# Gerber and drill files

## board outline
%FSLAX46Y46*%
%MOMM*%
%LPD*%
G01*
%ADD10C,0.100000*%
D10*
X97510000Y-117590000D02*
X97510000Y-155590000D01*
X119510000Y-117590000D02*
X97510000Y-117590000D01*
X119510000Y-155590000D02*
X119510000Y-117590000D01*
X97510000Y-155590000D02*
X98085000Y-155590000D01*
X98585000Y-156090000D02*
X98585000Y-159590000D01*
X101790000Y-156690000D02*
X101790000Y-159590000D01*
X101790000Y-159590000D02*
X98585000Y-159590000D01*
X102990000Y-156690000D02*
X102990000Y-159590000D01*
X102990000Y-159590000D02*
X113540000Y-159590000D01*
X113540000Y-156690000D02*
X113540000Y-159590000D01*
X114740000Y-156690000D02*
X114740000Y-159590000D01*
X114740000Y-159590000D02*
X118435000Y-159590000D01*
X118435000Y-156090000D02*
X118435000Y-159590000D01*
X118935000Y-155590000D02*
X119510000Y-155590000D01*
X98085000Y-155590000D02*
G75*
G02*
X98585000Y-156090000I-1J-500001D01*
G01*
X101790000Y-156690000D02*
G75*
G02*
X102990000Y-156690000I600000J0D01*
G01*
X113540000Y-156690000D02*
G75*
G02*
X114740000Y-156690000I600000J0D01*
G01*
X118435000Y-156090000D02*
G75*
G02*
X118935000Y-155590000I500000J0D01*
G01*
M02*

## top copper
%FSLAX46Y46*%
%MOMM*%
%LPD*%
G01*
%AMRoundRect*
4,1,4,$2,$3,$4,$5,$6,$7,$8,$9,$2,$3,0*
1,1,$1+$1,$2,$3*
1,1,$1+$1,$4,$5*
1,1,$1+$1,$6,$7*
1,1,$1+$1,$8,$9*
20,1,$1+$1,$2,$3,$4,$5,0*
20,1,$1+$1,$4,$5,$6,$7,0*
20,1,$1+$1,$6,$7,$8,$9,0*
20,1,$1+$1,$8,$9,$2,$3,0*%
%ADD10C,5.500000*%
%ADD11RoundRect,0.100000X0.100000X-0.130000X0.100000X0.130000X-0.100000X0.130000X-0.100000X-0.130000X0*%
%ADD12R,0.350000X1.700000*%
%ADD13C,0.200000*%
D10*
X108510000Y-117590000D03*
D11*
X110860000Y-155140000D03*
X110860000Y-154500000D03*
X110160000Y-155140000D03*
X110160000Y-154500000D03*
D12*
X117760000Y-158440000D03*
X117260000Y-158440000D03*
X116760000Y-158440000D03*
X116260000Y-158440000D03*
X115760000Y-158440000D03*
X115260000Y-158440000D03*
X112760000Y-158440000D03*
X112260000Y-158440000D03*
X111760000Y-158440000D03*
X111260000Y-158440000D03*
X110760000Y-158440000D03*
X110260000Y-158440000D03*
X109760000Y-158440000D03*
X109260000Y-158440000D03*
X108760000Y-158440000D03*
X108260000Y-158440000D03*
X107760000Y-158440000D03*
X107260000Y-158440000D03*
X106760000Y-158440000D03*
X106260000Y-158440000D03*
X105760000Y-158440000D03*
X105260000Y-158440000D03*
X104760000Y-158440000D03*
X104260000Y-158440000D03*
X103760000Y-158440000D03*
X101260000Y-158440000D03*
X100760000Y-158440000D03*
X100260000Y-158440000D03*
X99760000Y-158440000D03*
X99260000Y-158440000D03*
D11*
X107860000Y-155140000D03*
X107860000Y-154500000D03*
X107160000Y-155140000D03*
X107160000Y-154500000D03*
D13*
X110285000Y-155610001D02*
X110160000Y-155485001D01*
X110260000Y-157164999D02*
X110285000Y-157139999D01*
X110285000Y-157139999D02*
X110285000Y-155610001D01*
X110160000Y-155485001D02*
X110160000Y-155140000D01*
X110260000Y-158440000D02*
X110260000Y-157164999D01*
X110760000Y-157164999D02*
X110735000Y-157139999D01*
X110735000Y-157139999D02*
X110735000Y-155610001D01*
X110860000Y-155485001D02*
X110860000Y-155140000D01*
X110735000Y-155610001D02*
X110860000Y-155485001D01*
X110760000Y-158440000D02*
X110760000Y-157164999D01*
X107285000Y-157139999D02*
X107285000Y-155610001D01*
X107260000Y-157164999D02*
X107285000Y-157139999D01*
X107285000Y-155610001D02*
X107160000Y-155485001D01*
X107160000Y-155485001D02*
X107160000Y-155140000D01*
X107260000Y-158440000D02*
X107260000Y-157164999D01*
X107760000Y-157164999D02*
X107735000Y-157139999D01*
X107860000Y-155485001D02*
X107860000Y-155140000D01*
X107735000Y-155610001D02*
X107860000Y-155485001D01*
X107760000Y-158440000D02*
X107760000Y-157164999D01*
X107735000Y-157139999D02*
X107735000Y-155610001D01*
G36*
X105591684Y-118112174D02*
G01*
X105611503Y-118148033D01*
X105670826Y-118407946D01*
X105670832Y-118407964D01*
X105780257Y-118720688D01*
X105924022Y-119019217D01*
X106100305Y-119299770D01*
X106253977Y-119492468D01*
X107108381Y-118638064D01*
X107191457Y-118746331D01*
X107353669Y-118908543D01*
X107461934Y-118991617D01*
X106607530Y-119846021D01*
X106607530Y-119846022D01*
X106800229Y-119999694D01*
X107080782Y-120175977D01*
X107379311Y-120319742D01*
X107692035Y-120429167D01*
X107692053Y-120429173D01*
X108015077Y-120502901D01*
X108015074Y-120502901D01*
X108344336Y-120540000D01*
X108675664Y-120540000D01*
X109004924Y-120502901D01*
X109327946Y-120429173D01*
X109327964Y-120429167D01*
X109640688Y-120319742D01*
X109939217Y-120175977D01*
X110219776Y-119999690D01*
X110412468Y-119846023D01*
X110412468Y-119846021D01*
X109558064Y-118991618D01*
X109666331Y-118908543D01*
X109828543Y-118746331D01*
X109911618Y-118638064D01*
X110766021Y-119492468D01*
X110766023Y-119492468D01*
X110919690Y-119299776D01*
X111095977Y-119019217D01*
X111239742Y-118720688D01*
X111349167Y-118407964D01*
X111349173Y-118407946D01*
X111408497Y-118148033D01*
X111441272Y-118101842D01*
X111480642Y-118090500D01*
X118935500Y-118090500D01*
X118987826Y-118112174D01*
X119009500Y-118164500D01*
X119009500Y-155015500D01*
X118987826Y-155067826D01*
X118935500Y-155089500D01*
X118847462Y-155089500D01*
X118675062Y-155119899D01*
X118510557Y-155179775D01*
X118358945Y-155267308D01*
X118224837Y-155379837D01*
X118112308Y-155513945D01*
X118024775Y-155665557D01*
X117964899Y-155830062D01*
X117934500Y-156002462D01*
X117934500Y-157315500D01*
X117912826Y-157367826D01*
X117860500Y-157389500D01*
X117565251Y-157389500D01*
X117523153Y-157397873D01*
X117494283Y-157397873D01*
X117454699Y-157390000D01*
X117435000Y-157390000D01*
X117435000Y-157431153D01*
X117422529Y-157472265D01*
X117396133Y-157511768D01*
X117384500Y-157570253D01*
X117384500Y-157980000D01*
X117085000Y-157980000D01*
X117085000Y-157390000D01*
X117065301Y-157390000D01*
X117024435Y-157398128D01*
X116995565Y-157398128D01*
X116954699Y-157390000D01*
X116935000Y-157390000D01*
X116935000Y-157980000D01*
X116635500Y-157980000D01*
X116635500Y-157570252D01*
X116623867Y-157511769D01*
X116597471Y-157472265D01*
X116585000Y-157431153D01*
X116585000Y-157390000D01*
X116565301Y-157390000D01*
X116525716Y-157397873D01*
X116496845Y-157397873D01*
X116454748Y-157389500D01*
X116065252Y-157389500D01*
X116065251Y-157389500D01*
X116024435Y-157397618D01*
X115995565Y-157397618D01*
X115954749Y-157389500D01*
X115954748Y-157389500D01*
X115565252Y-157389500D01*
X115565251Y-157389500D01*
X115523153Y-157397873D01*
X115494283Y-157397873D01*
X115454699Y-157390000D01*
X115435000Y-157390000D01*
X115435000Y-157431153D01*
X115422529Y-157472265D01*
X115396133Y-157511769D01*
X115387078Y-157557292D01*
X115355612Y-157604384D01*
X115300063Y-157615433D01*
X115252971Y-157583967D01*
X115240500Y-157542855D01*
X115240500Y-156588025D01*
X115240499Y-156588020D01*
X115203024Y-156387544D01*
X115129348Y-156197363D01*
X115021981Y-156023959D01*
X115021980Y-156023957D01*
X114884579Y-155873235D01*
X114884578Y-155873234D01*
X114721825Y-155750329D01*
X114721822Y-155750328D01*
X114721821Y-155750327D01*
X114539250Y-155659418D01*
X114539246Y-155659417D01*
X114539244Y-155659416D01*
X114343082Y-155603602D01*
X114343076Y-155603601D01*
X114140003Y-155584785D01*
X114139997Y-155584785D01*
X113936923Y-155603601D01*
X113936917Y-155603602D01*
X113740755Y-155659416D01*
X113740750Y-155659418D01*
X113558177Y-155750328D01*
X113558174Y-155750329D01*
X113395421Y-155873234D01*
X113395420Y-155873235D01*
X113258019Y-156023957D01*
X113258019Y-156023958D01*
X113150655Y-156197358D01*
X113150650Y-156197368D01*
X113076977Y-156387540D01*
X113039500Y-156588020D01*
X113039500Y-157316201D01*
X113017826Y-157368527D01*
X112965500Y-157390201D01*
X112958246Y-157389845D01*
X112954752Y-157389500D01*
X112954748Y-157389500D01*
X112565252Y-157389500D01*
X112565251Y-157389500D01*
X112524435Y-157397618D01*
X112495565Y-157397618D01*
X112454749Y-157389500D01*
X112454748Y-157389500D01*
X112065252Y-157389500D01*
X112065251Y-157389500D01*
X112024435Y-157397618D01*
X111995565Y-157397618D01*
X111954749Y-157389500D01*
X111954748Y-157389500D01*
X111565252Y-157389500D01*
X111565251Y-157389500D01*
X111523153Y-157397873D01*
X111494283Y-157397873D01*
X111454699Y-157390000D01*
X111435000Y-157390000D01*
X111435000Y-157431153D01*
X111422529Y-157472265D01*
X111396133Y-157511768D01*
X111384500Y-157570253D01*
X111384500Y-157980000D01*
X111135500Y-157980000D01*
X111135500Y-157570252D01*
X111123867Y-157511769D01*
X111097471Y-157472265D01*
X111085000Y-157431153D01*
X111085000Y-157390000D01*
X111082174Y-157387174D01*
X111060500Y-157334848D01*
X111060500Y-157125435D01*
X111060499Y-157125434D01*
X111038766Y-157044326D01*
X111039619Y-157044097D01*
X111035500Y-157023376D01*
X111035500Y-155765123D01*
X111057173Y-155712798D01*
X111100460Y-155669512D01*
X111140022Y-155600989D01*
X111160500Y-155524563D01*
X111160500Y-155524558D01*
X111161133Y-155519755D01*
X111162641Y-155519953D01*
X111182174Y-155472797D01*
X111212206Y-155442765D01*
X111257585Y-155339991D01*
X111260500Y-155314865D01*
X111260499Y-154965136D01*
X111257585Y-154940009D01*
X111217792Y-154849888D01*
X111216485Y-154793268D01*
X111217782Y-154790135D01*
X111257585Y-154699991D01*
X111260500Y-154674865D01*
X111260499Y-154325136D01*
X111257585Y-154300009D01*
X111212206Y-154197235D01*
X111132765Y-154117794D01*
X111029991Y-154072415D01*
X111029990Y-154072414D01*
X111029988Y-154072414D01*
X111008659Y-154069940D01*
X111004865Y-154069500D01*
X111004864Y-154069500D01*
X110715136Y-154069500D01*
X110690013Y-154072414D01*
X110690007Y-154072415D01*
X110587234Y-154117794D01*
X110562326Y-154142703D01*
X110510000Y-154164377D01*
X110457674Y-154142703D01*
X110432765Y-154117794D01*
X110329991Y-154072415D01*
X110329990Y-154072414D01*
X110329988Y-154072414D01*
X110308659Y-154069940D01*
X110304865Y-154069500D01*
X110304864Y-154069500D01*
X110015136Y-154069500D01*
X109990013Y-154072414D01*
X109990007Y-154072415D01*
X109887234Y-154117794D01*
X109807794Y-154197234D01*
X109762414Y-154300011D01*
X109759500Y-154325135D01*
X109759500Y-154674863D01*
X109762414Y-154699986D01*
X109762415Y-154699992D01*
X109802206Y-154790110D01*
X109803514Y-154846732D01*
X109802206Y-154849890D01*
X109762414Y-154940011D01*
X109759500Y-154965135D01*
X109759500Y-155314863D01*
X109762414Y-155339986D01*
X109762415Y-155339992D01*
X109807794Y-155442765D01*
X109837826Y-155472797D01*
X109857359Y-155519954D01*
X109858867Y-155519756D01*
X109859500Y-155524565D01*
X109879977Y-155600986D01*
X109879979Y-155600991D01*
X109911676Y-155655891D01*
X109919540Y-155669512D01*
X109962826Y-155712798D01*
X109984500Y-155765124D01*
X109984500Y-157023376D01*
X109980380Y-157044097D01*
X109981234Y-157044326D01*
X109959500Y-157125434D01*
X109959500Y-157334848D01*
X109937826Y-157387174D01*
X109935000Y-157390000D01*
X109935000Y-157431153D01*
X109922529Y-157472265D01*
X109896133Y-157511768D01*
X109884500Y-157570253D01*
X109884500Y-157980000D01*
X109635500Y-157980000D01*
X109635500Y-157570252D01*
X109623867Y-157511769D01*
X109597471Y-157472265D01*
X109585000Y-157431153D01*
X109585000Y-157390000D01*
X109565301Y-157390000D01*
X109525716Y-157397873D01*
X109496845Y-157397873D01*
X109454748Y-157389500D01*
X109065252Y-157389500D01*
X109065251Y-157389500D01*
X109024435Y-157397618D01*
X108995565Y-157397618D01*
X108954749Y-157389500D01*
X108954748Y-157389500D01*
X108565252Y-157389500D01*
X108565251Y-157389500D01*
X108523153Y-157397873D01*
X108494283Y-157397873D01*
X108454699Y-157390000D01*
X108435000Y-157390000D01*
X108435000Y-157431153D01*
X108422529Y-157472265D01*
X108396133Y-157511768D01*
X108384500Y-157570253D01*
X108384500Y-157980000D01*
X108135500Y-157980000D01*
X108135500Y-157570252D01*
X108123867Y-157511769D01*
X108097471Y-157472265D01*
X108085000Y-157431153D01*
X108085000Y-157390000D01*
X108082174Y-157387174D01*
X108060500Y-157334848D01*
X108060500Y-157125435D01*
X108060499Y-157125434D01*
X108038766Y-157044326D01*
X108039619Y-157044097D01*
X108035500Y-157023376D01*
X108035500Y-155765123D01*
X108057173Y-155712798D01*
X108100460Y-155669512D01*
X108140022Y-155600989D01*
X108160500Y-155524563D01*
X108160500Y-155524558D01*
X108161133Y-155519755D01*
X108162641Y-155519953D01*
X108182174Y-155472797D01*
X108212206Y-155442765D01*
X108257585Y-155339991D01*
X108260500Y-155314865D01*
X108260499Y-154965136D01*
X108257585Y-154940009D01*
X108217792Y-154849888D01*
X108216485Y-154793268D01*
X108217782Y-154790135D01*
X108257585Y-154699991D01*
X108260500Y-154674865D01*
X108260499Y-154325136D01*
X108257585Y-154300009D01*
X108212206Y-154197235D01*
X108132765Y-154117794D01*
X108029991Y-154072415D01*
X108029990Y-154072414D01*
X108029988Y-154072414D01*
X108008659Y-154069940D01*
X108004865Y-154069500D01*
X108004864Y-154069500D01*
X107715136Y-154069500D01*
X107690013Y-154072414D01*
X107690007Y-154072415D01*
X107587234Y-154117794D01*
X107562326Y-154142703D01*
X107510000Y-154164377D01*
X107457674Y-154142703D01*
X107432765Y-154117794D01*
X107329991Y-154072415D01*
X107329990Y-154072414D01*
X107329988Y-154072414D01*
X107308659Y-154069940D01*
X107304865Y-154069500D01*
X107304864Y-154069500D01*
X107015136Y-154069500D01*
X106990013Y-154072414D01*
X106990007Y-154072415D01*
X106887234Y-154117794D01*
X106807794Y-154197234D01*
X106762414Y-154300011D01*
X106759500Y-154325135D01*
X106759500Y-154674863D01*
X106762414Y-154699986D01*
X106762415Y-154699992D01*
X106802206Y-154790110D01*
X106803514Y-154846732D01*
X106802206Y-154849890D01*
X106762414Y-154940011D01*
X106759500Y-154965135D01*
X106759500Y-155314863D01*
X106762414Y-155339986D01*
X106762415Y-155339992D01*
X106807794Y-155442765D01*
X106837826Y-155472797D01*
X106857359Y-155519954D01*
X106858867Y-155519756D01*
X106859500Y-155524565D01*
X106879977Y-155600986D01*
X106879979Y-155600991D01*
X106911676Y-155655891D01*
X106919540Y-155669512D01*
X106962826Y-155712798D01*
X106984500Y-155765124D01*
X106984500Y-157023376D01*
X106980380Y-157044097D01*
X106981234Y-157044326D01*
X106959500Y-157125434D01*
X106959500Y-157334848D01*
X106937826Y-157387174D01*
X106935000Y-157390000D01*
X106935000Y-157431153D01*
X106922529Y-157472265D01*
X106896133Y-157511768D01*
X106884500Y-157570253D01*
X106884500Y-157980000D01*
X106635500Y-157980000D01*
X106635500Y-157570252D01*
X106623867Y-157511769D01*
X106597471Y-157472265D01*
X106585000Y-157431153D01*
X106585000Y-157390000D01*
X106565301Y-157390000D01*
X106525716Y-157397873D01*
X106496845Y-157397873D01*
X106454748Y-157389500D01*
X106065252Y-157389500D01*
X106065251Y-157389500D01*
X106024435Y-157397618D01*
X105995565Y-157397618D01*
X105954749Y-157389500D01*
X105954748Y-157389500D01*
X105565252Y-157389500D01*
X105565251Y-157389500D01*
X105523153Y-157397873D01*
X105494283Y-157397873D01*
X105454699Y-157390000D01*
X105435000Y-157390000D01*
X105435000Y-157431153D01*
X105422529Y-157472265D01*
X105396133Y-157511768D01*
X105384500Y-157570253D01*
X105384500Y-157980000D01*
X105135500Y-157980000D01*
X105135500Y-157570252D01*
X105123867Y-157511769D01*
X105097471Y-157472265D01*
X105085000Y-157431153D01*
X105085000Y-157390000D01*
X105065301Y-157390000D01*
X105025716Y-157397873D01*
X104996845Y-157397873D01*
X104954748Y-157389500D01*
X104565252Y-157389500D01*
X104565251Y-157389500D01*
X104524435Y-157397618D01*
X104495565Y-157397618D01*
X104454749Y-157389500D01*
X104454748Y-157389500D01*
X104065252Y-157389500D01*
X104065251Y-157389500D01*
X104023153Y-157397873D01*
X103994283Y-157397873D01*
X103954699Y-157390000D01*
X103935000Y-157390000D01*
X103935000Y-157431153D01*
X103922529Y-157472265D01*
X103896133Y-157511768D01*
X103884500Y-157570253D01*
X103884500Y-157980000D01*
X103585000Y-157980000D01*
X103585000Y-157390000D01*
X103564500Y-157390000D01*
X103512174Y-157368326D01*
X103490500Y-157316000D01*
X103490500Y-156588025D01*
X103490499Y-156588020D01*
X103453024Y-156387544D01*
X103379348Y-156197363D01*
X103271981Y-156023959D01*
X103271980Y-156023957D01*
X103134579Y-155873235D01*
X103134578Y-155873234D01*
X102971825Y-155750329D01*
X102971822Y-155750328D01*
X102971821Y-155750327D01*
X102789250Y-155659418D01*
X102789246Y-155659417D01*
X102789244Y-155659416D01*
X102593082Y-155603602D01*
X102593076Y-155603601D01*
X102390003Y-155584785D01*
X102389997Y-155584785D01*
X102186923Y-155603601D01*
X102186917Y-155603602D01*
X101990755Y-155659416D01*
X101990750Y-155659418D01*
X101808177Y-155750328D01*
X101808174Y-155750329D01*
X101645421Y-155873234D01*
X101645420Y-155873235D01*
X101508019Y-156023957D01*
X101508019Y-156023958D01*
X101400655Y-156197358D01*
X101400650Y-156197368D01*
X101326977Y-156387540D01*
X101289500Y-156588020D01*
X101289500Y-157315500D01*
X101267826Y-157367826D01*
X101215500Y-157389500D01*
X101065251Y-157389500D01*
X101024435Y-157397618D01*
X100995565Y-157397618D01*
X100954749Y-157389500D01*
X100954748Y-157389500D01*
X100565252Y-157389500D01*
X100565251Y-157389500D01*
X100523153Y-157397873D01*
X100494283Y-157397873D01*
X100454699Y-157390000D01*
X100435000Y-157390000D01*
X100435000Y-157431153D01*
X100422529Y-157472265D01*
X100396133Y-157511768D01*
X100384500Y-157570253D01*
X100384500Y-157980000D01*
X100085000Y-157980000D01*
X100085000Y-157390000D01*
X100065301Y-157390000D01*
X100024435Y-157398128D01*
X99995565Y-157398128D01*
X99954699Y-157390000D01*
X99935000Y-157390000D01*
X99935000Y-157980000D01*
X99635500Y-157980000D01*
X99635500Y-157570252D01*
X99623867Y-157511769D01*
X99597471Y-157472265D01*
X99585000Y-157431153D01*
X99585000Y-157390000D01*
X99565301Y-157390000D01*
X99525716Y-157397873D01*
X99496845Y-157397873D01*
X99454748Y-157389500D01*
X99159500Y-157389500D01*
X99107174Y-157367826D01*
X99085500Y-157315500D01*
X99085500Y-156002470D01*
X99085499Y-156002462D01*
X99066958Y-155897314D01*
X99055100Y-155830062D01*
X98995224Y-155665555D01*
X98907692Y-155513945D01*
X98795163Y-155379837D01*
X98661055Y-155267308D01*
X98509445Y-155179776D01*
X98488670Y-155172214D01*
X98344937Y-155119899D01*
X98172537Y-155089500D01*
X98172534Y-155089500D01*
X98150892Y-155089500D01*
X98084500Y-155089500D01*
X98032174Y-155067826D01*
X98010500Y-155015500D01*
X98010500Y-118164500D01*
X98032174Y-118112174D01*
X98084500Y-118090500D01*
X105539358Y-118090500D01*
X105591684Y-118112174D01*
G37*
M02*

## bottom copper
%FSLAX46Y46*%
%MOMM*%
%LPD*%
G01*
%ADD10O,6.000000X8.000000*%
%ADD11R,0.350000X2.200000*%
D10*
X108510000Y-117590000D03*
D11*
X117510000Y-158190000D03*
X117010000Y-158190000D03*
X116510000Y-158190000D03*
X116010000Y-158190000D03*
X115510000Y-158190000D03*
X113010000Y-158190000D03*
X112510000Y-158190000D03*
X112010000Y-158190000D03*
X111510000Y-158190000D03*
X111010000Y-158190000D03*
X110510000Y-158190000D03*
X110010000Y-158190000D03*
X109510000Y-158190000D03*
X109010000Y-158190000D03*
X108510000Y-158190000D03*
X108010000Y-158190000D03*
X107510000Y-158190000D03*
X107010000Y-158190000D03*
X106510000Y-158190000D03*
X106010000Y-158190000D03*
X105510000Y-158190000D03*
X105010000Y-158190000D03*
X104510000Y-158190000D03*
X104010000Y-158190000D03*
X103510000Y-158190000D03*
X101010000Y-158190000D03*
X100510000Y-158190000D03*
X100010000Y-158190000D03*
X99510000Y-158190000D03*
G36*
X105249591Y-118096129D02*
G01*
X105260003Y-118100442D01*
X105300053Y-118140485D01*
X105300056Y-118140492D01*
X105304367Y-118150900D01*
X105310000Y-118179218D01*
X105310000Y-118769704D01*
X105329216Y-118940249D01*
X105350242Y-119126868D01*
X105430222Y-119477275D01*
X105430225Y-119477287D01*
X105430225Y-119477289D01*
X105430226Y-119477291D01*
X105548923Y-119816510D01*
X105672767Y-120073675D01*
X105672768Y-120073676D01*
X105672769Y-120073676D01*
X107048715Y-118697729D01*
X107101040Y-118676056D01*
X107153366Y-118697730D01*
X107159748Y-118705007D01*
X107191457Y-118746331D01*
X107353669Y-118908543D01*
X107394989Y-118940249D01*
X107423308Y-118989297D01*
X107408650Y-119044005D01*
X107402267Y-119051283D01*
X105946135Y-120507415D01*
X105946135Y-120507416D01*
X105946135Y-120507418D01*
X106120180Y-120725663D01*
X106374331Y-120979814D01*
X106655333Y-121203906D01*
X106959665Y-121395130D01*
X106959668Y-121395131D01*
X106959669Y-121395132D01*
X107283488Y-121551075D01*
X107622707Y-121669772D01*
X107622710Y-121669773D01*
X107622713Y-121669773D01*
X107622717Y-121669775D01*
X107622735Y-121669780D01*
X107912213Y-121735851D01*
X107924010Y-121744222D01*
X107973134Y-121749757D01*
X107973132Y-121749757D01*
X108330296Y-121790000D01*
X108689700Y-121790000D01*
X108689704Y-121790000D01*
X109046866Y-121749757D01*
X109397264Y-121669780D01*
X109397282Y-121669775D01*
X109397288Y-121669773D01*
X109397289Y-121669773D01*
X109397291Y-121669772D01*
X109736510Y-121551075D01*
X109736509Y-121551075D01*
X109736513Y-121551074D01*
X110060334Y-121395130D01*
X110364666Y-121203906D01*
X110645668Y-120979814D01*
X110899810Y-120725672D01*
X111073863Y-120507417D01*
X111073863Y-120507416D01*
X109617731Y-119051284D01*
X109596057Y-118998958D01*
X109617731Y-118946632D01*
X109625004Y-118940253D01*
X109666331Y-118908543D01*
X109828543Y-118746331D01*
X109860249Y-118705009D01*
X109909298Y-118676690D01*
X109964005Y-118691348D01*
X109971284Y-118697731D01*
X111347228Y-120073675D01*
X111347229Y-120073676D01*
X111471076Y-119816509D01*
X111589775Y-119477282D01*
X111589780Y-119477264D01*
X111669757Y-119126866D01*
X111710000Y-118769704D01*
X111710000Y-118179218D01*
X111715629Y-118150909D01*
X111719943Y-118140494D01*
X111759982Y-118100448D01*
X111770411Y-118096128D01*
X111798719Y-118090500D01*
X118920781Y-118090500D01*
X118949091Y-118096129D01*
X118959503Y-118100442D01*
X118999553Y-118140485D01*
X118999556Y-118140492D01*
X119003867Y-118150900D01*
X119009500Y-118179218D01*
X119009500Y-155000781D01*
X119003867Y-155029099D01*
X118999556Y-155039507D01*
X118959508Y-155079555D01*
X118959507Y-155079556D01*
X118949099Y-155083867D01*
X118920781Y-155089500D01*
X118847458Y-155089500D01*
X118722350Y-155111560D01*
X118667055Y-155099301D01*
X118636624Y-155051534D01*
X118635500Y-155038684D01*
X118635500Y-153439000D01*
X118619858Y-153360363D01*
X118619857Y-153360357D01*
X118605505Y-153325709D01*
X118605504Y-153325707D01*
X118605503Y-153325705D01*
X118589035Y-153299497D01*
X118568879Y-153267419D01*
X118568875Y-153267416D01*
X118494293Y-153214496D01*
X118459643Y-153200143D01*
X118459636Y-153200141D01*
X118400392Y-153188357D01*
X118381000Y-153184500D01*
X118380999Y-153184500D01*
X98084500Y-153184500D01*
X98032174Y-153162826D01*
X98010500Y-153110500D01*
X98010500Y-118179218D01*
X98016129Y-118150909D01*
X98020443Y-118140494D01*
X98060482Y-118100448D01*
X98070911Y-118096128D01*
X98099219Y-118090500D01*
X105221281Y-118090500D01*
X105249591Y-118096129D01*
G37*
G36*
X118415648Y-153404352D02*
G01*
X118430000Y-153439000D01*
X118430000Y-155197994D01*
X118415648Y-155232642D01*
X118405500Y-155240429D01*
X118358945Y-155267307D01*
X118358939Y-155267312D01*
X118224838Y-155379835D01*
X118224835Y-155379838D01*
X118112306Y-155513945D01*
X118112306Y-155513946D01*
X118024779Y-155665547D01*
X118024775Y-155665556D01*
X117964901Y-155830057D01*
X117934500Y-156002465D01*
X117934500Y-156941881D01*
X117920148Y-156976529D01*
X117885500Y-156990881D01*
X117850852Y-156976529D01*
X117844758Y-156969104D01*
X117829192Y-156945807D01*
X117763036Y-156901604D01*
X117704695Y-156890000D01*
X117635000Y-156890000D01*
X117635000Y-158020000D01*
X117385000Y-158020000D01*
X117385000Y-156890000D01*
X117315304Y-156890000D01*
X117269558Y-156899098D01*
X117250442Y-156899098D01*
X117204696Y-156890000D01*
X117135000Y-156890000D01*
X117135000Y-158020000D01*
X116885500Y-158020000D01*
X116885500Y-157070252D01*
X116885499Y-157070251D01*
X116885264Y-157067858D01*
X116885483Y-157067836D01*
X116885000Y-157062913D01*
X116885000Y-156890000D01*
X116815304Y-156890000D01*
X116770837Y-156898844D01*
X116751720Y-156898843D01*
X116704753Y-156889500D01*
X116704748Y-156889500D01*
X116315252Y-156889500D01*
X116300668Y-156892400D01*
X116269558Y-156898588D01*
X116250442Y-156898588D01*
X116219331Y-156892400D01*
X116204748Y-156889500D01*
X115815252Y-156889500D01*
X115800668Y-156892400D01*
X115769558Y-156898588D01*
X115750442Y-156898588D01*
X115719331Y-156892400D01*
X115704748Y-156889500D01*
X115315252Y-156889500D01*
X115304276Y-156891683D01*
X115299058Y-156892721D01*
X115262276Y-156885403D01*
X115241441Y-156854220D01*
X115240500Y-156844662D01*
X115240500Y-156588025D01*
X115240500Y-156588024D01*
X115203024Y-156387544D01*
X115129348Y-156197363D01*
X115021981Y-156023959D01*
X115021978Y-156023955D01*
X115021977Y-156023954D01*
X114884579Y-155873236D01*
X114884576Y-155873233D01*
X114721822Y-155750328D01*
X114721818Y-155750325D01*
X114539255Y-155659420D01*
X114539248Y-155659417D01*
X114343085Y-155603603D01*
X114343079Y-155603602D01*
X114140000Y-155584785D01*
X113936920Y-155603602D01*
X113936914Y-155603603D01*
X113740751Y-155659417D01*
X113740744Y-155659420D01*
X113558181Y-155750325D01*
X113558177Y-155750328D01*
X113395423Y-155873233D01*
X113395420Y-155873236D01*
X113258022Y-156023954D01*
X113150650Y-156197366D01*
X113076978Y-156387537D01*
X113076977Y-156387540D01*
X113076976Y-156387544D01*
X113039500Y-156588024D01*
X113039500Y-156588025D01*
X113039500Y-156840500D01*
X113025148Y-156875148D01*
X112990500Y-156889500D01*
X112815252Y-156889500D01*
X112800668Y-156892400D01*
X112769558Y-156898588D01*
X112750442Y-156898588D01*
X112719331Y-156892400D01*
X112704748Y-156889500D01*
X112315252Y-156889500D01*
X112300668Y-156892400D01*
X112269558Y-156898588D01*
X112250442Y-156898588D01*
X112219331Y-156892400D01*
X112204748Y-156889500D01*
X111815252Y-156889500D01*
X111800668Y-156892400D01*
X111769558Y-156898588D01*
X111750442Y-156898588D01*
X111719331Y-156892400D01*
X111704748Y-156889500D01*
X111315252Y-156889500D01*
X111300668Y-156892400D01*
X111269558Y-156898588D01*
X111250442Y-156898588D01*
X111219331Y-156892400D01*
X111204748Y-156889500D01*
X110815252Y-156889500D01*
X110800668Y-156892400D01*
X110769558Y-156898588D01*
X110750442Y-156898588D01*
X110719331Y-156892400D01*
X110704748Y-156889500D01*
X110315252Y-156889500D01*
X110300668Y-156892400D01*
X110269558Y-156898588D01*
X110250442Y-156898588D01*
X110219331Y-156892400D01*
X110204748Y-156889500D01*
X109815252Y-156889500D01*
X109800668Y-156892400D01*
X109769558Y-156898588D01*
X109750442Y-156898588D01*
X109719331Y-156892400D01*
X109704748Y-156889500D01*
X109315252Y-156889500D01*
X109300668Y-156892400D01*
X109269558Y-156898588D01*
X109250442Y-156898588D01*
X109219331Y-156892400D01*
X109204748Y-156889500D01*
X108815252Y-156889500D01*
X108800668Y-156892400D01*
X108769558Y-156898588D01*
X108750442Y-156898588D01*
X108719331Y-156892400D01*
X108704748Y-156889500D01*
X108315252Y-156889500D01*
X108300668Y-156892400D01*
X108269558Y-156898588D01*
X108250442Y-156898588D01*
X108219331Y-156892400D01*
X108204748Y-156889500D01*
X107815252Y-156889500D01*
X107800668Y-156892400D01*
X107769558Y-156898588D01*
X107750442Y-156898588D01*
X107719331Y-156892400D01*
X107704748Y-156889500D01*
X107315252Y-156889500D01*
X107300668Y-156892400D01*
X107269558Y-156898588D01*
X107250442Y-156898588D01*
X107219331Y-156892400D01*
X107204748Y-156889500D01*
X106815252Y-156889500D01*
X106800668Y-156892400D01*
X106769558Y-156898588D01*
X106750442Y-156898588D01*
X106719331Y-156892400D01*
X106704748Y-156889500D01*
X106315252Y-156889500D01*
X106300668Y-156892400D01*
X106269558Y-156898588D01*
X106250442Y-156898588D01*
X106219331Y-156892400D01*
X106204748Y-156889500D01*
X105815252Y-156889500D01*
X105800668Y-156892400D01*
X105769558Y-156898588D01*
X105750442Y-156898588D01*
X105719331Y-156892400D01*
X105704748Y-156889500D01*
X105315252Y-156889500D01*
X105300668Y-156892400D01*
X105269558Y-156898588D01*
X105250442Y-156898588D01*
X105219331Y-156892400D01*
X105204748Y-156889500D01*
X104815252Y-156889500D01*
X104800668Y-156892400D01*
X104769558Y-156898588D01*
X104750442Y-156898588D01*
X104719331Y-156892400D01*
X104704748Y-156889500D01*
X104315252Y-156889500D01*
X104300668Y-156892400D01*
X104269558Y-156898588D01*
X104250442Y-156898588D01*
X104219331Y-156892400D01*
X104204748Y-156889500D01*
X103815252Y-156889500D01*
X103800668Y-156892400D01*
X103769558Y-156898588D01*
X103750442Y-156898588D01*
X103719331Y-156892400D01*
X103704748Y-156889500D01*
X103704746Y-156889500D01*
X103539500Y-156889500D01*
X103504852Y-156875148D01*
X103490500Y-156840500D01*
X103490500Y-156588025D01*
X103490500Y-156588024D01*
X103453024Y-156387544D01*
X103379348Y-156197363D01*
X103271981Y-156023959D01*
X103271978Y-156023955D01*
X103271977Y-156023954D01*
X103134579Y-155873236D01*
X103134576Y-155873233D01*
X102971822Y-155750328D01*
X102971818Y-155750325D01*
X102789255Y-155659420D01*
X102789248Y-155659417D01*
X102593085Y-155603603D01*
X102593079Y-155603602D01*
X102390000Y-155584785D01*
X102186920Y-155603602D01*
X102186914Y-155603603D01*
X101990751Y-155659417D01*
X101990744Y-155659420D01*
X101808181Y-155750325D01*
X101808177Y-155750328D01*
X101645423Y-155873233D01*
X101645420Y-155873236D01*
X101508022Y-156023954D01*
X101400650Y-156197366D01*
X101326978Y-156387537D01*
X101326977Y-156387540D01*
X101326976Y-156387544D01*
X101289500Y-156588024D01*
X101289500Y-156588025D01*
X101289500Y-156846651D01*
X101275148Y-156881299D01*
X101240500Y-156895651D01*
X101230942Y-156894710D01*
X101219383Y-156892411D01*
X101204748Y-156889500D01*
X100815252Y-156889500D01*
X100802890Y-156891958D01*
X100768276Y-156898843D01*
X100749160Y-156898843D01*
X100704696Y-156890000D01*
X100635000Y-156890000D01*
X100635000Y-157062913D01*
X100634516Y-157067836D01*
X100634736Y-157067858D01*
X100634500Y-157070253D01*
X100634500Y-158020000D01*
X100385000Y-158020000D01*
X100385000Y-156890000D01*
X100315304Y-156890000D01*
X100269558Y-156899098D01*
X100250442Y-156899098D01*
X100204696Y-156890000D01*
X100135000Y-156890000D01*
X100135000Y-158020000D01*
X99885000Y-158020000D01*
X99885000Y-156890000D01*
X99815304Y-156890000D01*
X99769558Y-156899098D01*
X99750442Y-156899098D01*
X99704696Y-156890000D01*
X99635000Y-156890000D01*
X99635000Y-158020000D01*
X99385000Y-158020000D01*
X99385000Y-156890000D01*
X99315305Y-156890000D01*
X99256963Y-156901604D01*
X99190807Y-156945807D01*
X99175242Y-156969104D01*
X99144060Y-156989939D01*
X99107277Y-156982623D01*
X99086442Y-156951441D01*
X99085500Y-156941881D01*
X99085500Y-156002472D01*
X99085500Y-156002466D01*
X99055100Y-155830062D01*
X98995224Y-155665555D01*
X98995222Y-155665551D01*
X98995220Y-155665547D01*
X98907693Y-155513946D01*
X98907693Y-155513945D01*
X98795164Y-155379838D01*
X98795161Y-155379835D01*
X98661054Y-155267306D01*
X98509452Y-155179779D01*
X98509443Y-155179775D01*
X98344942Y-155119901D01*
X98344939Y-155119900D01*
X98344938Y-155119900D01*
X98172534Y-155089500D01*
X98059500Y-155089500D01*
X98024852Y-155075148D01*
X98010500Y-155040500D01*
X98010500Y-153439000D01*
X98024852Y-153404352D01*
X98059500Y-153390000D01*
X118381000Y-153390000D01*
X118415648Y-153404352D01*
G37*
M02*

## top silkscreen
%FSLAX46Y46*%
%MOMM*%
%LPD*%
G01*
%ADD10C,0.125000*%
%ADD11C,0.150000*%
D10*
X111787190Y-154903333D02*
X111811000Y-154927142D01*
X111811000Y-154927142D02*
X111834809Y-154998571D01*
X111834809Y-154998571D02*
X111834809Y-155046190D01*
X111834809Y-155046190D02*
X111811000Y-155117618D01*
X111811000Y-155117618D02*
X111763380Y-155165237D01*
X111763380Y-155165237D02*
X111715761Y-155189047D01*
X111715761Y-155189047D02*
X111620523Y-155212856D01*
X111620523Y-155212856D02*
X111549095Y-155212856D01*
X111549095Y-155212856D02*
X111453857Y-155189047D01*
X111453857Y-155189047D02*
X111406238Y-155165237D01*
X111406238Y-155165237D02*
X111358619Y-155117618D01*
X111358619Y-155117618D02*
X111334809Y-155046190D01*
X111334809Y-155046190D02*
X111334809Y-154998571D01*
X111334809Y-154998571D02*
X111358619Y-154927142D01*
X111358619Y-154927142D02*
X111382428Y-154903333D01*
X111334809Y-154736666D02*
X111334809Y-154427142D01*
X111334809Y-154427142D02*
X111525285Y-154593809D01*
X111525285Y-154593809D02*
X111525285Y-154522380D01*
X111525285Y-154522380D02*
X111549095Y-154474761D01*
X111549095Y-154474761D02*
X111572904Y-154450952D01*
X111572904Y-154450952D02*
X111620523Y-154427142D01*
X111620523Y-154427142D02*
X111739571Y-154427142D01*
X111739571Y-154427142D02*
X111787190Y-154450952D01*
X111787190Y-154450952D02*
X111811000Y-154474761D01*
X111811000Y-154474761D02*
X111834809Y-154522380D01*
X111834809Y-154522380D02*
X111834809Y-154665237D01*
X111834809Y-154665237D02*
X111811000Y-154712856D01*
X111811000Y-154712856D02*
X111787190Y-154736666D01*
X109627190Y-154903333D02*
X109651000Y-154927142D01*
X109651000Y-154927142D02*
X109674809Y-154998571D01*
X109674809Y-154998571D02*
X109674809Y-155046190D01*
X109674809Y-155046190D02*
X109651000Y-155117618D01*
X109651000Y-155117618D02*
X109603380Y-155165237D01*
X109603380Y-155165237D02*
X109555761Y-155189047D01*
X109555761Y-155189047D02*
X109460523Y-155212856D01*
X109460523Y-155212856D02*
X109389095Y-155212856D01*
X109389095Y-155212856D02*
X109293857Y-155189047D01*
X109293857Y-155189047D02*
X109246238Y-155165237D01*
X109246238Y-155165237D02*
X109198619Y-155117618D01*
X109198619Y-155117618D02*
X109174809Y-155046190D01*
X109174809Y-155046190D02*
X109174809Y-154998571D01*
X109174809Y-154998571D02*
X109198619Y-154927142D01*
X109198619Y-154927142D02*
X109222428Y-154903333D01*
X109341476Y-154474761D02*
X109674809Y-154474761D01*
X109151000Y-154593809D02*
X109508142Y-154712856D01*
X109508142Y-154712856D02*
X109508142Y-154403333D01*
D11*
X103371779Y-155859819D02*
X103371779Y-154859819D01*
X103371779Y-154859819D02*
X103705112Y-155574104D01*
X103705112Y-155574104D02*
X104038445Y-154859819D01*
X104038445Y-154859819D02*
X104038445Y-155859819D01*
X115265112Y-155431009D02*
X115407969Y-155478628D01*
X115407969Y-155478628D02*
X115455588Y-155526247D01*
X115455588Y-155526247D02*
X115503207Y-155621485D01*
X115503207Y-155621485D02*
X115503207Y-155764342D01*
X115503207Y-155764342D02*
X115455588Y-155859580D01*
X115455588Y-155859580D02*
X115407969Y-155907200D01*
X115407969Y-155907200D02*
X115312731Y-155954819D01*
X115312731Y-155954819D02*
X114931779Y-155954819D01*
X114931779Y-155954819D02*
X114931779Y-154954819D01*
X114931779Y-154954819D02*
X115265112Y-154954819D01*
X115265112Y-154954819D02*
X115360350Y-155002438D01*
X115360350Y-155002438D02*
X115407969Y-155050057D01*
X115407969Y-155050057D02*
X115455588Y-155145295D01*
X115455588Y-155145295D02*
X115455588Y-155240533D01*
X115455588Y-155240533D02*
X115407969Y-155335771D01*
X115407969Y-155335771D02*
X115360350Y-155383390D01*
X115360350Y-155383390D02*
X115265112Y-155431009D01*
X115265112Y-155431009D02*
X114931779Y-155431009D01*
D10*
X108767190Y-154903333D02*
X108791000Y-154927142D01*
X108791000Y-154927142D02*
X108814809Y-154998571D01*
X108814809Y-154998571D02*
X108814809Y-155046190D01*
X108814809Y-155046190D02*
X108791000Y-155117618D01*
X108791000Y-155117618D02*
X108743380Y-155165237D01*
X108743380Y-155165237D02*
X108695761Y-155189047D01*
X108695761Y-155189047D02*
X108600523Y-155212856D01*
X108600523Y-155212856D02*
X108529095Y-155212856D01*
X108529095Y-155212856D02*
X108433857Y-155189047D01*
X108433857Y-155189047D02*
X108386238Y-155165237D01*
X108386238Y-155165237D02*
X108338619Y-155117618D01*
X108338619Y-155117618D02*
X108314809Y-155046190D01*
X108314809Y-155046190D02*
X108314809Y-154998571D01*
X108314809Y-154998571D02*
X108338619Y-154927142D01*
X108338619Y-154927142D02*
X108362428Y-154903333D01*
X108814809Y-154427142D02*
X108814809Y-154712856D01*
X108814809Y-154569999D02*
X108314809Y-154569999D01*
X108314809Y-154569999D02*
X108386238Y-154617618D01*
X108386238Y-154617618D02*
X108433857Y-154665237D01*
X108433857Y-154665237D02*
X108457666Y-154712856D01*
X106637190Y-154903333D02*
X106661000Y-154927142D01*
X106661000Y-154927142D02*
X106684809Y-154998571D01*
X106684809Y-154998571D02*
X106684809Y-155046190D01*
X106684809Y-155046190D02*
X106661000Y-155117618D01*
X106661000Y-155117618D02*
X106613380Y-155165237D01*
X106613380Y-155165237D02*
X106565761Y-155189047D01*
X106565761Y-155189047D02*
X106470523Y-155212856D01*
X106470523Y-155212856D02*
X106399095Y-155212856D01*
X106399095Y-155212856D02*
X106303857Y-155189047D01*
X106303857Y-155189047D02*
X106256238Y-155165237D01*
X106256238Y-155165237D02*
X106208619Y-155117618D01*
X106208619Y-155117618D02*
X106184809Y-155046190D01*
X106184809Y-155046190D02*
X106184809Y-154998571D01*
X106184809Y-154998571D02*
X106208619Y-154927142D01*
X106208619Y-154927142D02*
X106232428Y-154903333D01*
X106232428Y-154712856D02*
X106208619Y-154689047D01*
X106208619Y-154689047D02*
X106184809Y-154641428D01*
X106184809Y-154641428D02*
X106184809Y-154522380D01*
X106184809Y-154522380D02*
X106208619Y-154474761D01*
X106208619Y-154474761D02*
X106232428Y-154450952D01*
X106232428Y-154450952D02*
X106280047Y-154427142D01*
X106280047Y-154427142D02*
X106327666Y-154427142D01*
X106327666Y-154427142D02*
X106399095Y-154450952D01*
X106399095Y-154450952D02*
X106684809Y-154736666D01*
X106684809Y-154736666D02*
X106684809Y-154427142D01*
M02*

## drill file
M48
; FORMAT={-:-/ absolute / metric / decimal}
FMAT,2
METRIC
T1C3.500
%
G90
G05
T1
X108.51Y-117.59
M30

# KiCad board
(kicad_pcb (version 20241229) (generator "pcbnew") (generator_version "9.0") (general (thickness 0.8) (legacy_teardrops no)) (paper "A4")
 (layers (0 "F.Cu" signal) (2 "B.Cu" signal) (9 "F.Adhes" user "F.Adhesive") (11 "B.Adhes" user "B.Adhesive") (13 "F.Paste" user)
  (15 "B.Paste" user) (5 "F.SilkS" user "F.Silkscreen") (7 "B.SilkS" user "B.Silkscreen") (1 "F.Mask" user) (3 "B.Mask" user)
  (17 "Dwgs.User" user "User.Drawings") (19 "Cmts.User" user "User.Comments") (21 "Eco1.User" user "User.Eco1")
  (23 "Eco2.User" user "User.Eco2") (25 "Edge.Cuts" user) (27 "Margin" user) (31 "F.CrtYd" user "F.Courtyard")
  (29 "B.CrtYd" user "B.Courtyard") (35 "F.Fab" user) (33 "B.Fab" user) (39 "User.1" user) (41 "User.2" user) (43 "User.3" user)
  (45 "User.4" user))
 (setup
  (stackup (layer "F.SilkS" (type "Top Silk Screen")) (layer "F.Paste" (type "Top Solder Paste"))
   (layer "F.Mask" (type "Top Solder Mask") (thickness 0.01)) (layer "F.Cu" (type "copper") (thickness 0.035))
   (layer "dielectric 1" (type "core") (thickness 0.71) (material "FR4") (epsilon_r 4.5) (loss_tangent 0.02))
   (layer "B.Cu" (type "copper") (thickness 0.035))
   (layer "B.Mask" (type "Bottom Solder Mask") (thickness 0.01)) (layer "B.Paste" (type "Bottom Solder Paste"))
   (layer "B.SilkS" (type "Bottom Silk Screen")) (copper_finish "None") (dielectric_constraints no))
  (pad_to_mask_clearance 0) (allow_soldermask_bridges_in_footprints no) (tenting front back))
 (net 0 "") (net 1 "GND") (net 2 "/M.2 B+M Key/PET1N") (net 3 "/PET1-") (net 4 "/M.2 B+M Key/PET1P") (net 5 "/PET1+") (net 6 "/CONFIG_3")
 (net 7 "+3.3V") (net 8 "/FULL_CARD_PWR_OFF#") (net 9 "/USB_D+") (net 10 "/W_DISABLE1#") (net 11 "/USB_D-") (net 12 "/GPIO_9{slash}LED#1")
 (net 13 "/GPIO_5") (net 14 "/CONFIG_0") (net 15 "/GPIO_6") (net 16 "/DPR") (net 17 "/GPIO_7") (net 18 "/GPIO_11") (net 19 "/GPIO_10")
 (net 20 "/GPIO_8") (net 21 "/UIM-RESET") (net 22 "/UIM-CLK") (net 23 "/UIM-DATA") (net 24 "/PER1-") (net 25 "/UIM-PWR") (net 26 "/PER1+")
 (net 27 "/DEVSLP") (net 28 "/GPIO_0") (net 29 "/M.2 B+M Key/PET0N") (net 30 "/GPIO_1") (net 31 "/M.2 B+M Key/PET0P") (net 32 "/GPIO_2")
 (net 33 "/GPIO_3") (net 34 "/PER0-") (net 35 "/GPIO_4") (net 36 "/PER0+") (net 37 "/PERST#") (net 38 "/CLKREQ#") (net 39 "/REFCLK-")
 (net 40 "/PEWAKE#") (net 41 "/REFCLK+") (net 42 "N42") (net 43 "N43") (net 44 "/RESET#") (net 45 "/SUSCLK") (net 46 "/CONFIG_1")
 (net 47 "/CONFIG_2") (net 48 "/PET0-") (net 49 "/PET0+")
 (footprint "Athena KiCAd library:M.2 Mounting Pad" (layer "F.Cu") (at 108.51 117.59)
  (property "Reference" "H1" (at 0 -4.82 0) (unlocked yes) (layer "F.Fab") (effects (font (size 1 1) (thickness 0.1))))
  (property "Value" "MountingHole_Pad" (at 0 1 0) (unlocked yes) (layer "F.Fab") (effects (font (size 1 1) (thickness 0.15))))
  (pad "1" thru_hole circle (at 0 0) (size 5.5 5.5) (drill 3.5) (layers "*.Cu" "*.Mask") (remove_unused_layers no) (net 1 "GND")
   (padstack (mode front_inner_back)
    (layer "Inner" (shape circle) (size 5.5 5.5) (zone_connect -1))
    (layer "B.Cu" (shape oval) (size 6 8) (thermal_bridge_angle 45) (zone_connect -1)))))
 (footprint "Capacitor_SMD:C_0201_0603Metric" (layer "F.Cu") (at 110.86 154.82 90)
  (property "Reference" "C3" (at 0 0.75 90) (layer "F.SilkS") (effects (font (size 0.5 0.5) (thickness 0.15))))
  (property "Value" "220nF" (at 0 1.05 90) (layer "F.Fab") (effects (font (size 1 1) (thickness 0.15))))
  (pad "" smd roundrect (at -0.345 0 90) (size 0.318 0.36) (layers "F.Paste") (roundrect_rratio 0.25))
  (pad "" smd roundrect (at 0.345 0 90) (size 0.318 0.36) (layers "F.Paste") (roundrect_rratio 0.25))
  (pad "1" smd roundrect (at -0.32 0 90) (size 0.46 0.4) (layers "F.Cu" "F.Mask") (roundrect_rratio 0.25) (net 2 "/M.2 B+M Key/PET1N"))
  (pad "2" smd roundrect (at 0.32 0 90) (size 0.46 0.4) (layers "F.Cu" "F.Mask") (roundrect_rratio 0.25) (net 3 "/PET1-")))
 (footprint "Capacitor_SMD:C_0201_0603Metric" (layer "F.Cu") (at 110.16 154.82 90)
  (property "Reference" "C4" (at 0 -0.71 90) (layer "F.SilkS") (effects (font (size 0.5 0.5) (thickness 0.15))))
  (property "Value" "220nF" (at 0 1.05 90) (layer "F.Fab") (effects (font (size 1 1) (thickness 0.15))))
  (pad "" smd roundrect (at -0.345 0 90) (size 0.318 0.36) (layers "F.Paste") (roundrect_rratio 0.25))
  (pad "" smd roundrect (at 0.345 0 90) (size 0.318 0.36) (layers "F.Paste") (roundrect_rratio 0.25))
  (pad "1" smd roundrect (at -0.32 0 90) (size 0.46 0.4) (layers "F.Cu" "F.Mask") (roundrect_rratio 0.25) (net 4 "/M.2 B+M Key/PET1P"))
  (pad "2" smd roundrect (at 0.32 0 90) (size 0.46 0.4) (layers "F.Cu" "F.Mask") (roundrect_rratio 0.25) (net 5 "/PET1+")))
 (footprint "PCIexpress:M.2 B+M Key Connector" (layer "F.Cu") (at 108.51 158.48)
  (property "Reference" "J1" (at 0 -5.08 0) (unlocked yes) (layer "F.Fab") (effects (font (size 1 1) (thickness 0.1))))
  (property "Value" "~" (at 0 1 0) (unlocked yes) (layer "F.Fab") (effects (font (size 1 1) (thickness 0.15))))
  (fp_line (start -11 -2.89) (end -10.425 -2.89) (stroke (width 0.1) (type default)) (layer "Edge.Cuts") (net 4))
  (fp_line (start -9.925 -2.39) (end -9.925 1.11) (stroke (width 0.1) (type default)) (layer "Edge.Cuts") (net 4))
  (fp_line (start -6.72 -1.79) (end -6.72 1.11) (stroke (width 0.1) (type default)) (layer "Edge.Cuts") (net 4))
  (fp_line (start -6.72 1.11) (end -9.925 1.11) (stroke (width 0.1) (type default)) (layer "Edge.Cuts") (net 4))
  (fp_line (start -5.52 -1.79) (end -5.52 1.11) (stroke (width 0.1) (type default)) (layer "Edge.Cuts") (net 4))
  (fp_line (start -5.52 1.11) (end 5.03 1.11) (stroke (width 0.1) (type default)) (layer "Edge.Cuts") (net 4))
  (fp_line (start 5.03 -1.79) (end 5.03 1.11) (stroke (width 0.1) (type default)) (layer "Edge.Cuts") (net 4))
  (fp_line (start 6.23 -1.79) (end 6.23 1.11) (stroke (width 0.1) (type default)) (layer "Edge.Cuts") (net 4))
  (fp_line (start 6.23 1.11) (end 9.925 1.11) (stroke (width 0.1) (type default)) (layer "Edge.Cuts") (net 4))
  (fp_line (start 9.925 -2.39) (end 9.925 1.11) (stroke (width 0.1) (type default)) (layer "Edge.Cuts") (net 4))
  (fp_line (start 10.425 -2.89) (end 11 -2.89) (stroke (width 0.1) (type default)) (layer "Edge.Cuts") (net 4))
  (fp_arc (start -10.425 -2.89) (mid -10.071447 -2.743553) (end -9.925 -2.39) (stroke (width 0.1) (type default)) (layer "Edge.Cuts")
   (net 4))
  (fp_arc (start -6.72 -1.79) (mid -6.12 -2.39) (end -5.52 -1.79) (stroke (width 0.1) (type default)) (layer "Edge.Cuts") (net 4))
  (fp_arc (start 5.03 -1.79) (mid 5.63 -2.39) (end 6.23 -1.79) (stroke (width 0.1) (type default)) (layer "Edge.Cuts") (net 4))
  (fp_arc (start 9.925 -2.39) (mid 10.071447 -2.743553) (end 10.425 -2.89) (stroke (width 0.1) (type default)) (layer "Edge.Cuts") (net 4))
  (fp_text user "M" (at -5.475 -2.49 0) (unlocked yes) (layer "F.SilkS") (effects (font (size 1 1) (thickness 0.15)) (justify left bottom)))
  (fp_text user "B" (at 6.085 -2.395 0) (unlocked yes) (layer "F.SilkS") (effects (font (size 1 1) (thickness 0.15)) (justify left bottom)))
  (pad "1" smd rect (at 9.25 -0.04 180) (size 0.35 1.7) (layers "F.Cu") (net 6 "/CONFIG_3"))
  (pad "2" smd rect (at 9 -0.29 180) (size 0.35 2.2) (layers "B.Cu") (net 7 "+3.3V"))
  (pad "3" smd rect (at 8.75 -0.04 180) (size 0.35 1.7) (layers "F.Cu") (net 1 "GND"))
  (pad "4" smd rect (at 8.5 -0.29 180) (size 0.35 2.2) (layers "B.Cu") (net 7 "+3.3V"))
  (pad "5" smd rect (at 8.25 -0.04 180) (size 0.35 1.7) (layers "F.Cu") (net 1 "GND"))
  (pad "6" smd rect (at 8 -0.29 180) (size 0.35 2.2) (layers "B.Cu") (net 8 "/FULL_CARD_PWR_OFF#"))
  (pad "7" smd rect (at 7.75 -0.04 180) (size 0.35 1.7) (layers "F.Cu") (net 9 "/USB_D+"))
  (pad "8" smd rect (at 7.5 -0.29 180) (size 0.35 2.2) (layers "B.Cu") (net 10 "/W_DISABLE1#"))
  (pad "9" smd rect (at 7.25 -0.04 180) (size 0.35 1.7) (layers "F.Cu") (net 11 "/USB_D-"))
  (pad "10" smd rect (at 7 -0.29 180) (size 0.35 2.2) (layers "B.Cu") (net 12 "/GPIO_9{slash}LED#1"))
  (pad "11" smd rect (at 6.75 -0.04 180) (size 0.35 1.7) (layers "F.Cu") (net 1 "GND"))
  (pad "20" smd rect (at 4.5 -0.29 180) (size 0.35 2.2) (layers "B.Cu") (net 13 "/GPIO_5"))
  (pad "21" smd rect (at 4.25 -0.04 180) (size 0.35 1.7) (layers "F.Cu") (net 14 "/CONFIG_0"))
  (pad "22" smd rect (at 4 -0.29 180) (size 0.35 2.2) (layers "B.Cu") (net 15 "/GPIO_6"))
  (pad "23" smd rect (at 3.75 -0.04 180) (size 0.35 1.7) (layers "F.Cu") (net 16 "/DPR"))
  (pad "24" smd rect (at 3.5 -0.29 180) (size 0.35 2.2) (layers "B.Cu") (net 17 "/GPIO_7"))
  (pad "25" smd rect (at 3.25 -0.04 180) (size 0.35 1.7) (layers "F.Cu") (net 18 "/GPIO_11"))
  (pad "26" smd rect (at 3 -0.29 180) (size 0.35 2.2) (layers "B.Cu") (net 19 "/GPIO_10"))
  (pad "27" smd rect (at 2.75 -0.04 180) (size 0.35 1.7) (layers "F.Cu") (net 1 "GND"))
  (pad "28" smd rect (at 2.5 -0.29 180) (size 0.35 2.2) (layers "B.Cu") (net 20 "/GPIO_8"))
  (pad "29" smd rect (at 2.25 -0.04 180) (size 0.35 1.7) (layers "F.Cu") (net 2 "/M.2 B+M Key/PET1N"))
  (pad "30" smd rect (at 2 -0.29 180) (size 0.35 2.2) (layers "B.Cu") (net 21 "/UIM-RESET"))
  (pad "31" smd rect (at 1.75 -0.04 180) (size 0.35 1.7) (layers "F.Cu") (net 4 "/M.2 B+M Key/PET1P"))
  (pad "32" smd rect (at 1.5 -0.29 180) (size 0.35 2.2) (layers "B.Cu") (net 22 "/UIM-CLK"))
  (pad "33" smd rect (at 1.25 -0.04 180) (size 0.35 1.7) (layers "F.Cu") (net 1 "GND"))
  (pad "34" smd rect (at 1 -0.29 180) (size 0.35 2.2) (layers "B.Cu") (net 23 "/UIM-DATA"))
  (pad "35" smd rect (at 0.75 -0.04 180) (size 0.35 1.7) (layers "F.Cu") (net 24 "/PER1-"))
  (pad "36" smd rect (at 0.5 -0.29 180) (size 0.35 2.2) (layers "B.Cu") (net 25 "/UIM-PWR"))
  (pad "37" smd rect (at 0.25 -0.04 180) (size 0.35 1.7) (layers "F.Cu") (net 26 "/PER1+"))
  (pad "38" smd rect (at 0 -0.29 180) (size 0.35 2.2) (layers "B.Cu") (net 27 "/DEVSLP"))
  (pad "39" smd rect (at -0.25 -0.04 180) (size 0.35 1.7) (layers "F.Cu") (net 1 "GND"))
  (pad "40" smd rect (at -0.5 -0.29 180) (size 0.35 2.2) (layers "B.Cu") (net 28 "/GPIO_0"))
  (pad "41" smd rect (at -0.75 -0.04 180) (size 0.35 1.7) (layers "F.Cu") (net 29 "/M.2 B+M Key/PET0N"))
  (pad "42" smd rect (at -1 -0.29 180) (size 0.35 2.2) (layers "B.Cu") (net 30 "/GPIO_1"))
  (pad "43" smd rect (at -1.25 -0.04 180) (size 0.35 1.7) (layers "F.Cu") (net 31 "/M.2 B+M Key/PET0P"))
  (pad "44" smd rect (at -1.5 -0.29 180) (size 0.35 2.2) (layers "B.Cu") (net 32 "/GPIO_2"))
  (pad "45" smd rect (at -1.75 -0.04 180) (size 0.35 1.7) (layers "F.Cu") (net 1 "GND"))
  (pad "46" smd rect (at -2 -0.29 180) (size 0.35 2.2) (layers "B.Cu") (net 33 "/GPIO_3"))
  (pad "47" smd rect (at -2.25 -0.04 180) (size 0.35 1.7) (layers "F.Cu") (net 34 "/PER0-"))
  (pad "48" smd rect (at -2.5 -0.29 180) (size 0.35 2.2) (layers "B.Cu") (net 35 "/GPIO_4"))
  (pad "49" smd rect (at -2.75 -0.04 180) (size 0.35 1.7) (layers "F.Cu") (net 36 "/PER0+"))
  (pad "50" smd rect (at -3 -0.29 180) (size 0.35 2.2) (layers "B.Cu") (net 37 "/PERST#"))
  (pad "51" smd rect (at -3.25 -0.04 180) (size 0.35 1.7) (layers "F.Cu") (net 1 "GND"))
  (pad "52" smd rect (at -3.5 -0.29 180) (size 0.35 2.2) (layers "B.Cu") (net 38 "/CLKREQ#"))
  (pad "53" smd rect (at -3.75 -0.04 180) (size 0.35 1.7) (layers "F.Cu") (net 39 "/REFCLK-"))
  (pad "54" smd rect (at -4 -0.29 180) (size 0.35 2.2) (layers "B.Cu") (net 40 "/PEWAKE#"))
  (pad "55" smd rect (at -4.25 -0.04 180) (size 0.35 1.7) (layers "F.Cu") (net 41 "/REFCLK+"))
  (pad "56" smd rect (at -4.5 -0.29 180) (size 0.35 2.2) (layers "B.Cu") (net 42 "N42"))
  (pad "57" smd rect (at -4.75 -0.04 180) (size 0.35 1.7) (layers "F.Cu") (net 1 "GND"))
  (pad "58" smd rect (at -5 -0.29 180) (size 0.35 2.2) (layers "B.Cu") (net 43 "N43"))
  (pad "67" smd rect (at -7.25 -0.04 180) (size 0.35 1.7) (layers "F.Cu") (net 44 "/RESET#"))
  (pad "68" smd rect (at -7.5 -0.29 180) (size 0.35 2.2) (layers "B.Cu") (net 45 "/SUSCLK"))
  (pad "69" smd rect (at -7.75 -0.04 180) (size 0.35 1.7) (layers "F.Cu") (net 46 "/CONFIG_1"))
  (pad "70" smd rect (at -8 -0.29 180) (size 0.35 2.2) (layers "B.Cu") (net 7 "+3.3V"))
  (pad "71" smd rect (at -8.25 -0.04 180) (size 0.35 1.7) (layers "F.Cu") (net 1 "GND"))
  (pad "72" smd rect (at -8.5 -0.29 180) (size 0.35 2.2) (layers "B.Cu") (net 7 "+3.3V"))
  (pad "73" smd rect (at -8.75 -0.04 180) (size 0.35 1.7) (layers "F.Cu") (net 1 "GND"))
  (pad "74" smd rect (at -9 -0.29 180) (size 0.35 2.2) (layers "B.Cu") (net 7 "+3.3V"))
  (pad "75" smd rect (at -9.25 -0.04 180) (size 0.35 1.7) (layers "F.Cu") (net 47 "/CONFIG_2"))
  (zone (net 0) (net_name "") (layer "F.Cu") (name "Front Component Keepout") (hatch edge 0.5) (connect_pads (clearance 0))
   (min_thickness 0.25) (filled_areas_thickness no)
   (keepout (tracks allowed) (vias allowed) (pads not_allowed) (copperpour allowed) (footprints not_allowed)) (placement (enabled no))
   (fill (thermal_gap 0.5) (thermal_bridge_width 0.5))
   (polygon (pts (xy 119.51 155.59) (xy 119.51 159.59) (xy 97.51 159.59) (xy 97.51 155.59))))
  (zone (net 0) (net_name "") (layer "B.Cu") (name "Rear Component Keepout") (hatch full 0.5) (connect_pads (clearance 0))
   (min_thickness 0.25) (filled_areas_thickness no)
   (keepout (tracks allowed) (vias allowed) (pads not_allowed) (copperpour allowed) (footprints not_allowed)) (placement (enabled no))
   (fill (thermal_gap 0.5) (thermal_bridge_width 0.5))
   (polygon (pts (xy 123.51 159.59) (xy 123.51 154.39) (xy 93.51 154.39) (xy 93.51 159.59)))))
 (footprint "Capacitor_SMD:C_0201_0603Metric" (layer "F.Cu") (at 107.86 154.82 90)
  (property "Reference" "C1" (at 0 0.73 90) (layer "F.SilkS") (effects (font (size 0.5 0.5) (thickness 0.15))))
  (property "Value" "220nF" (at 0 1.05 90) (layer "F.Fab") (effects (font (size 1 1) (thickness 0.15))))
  (pad "" smd roundrect (at -0.345 0 90) (size 0.318 0.36) (layers "F.Paste") (roundrect_rratio 0.25))
  (pad "" smd roundrect (at 0.345 0 90) (size 0.318 0.36) (layers "F.Paste") (roundrect_rratio 0.25))
  (pad "1" smd roundrect (at -0.32 0 90) (size 0.46 0.4) (layers "F.Cu" "F.Mask") (roundrect_rratio 0.25) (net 29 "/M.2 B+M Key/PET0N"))
  (pad "2" smd roundrect (at 0.32 0 90) (size 0.46 0.4) (layers "F.Cu" "F.Mask") (roundrect_rratio 0.25) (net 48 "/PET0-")))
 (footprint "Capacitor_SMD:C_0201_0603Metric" (layer "F.Cu") (at 107.16 154.82 90)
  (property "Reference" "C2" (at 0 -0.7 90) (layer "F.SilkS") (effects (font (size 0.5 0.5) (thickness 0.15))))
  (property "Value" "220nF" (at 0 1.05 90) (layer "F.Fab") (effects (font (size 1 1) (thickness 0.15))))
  (pad "" smd roundrect (at -0.345 0 90) (size 0.318 0.36) (layers "F.Paste") (roundrect_rratio 0.25))
  (pad "" smd roundrect (at 0.345 0 90) (size 0.318 0.36) (layers "F.Paste") (roundrect_rratio 0.25))
  (pad "1" smd roundrect (at -0.32 0 90) (size 0.46 0.4) (layers "F.Cu" "F.Mask") (roundrect_rratio 0.25) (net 31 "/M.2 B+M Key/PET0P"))
  (pad "2" smd roundrect (at 0.32 0 90) (size 0.46 0.4) (layers "F.Cu" "F.Mask") (roundrect_rratio 0.25) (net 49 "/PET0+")))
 (gr_line (start 97.51 117.59) (end 97.51 155.59) (stroke (width 0.1) (type default)) (layer "Edge.Cuts"))
 (gr_line (start 119.51 117.59) (end 97.51 117.59) (stroke (width 0.1) (type default)) (layer "Edge.Cuts"))
 (gr_line (start 119.51 155.59) (end 119.51 117.59) (stroke (width 0.1) (type default)) (layer "Edge.Cuts"))
 (segment (start 110.285 155.610001) (end 110.16 155.485001) (width 0.2) (layer "F.Cu") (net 4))
 (segment (start 110.26 157.164999) (end 110.285 157.139999) (width 0.2) (layer "F.Cu") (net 4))
 (segment (start 110.285 157.139999) (end 110.285 155.610001) (width 0.2) (layer "F.Cu") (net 4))
 (segment (start 110.16 155.485001) (end 110.16 155.14) (width 0.2) (layer "F.Cu") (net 4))
 (segment (start 110.26 158.44) (end 110.26 157.164999) (width 0.2) (layer "F.Cu") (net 4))
 (segment (start 110.76 157.164999) (end 110.735 157.139999) (width 0.2) (layer "F.Cu") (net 2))
 (segment (start 110.735 157.139999) (end 110.735 155.610001) (width 0.2) (layer "F.Cu") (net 2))
 (segment (start 110.86 155.485001) (end 110.86 155.14) (width 0.2) (layer "F.Cu") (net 2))
 (segment (start 110.735 155.610001) (end 110.86 155.485001) (width 0.2) (layer "F.Cu") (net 2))
 (segment (start 110.76 158.44) (end 110.76 157.164999) (width 0.2) (layer "F.Cu") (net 2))
 (segment (start 107.285 157.139999) (end 107.285 155.610001) (width 0.2) (layer "F.Cu") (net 31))
 (segment (start 107.26 157.164999) (end 107.285 157.139999) (width 0.2) (layer "F.Cu") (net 31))
 (segment (start 107.285 155.610001) (end 107.16 155.485001) (width 0.2) (layer "F.Cu") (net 31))
 (segment (start 107.16 155.485001) (end 107.16 155.14) (width 0.2) (layer "F.Cu") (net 31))
 (segment (start 107.26 158.44) (end 107.26 157.164999) (width 0.2) (layer "F.Cu") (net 31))
 (segment (start 107.76 157.164999) (end 107.735 157.139999) (width 0.2) (layer "F.Cu") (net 29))
 (segment (start 107.86 155.485001) (end 107.86 155.14) (width 0.2) (layer "F.Cu") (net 29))
 (segment (start 107.735 155.610001) (end 107.86 155.485001) (width 0.2) (layer "F.Cu") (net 29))
 (segment (start 107.76 158.44) (end 107.76 157.164999) (width 0.2) (layer "F.Cu") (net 29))
 (segment (start 107.735 157.139999) (end 107.735 155.610001) (width 0.2) (layer "F.Cu") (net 29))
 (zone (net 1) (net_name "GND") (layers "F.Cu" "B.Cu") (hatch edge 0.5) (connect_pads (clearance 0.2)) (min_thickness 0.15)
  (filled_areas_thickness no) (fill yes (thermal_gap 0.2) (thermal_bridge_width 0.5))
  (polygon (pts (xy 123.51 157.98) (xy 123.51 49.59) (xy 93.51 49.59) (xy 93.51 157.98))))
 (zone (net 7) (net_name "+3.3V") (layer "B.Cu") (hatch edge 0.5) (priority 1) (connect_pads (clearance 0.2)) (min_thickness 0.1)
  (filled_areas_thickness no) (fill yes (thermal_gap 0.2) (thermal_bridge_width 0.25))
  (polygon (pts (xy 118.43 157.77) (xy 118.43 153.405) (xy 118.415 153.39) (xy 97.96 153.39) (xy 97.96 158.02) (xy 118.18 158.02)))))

